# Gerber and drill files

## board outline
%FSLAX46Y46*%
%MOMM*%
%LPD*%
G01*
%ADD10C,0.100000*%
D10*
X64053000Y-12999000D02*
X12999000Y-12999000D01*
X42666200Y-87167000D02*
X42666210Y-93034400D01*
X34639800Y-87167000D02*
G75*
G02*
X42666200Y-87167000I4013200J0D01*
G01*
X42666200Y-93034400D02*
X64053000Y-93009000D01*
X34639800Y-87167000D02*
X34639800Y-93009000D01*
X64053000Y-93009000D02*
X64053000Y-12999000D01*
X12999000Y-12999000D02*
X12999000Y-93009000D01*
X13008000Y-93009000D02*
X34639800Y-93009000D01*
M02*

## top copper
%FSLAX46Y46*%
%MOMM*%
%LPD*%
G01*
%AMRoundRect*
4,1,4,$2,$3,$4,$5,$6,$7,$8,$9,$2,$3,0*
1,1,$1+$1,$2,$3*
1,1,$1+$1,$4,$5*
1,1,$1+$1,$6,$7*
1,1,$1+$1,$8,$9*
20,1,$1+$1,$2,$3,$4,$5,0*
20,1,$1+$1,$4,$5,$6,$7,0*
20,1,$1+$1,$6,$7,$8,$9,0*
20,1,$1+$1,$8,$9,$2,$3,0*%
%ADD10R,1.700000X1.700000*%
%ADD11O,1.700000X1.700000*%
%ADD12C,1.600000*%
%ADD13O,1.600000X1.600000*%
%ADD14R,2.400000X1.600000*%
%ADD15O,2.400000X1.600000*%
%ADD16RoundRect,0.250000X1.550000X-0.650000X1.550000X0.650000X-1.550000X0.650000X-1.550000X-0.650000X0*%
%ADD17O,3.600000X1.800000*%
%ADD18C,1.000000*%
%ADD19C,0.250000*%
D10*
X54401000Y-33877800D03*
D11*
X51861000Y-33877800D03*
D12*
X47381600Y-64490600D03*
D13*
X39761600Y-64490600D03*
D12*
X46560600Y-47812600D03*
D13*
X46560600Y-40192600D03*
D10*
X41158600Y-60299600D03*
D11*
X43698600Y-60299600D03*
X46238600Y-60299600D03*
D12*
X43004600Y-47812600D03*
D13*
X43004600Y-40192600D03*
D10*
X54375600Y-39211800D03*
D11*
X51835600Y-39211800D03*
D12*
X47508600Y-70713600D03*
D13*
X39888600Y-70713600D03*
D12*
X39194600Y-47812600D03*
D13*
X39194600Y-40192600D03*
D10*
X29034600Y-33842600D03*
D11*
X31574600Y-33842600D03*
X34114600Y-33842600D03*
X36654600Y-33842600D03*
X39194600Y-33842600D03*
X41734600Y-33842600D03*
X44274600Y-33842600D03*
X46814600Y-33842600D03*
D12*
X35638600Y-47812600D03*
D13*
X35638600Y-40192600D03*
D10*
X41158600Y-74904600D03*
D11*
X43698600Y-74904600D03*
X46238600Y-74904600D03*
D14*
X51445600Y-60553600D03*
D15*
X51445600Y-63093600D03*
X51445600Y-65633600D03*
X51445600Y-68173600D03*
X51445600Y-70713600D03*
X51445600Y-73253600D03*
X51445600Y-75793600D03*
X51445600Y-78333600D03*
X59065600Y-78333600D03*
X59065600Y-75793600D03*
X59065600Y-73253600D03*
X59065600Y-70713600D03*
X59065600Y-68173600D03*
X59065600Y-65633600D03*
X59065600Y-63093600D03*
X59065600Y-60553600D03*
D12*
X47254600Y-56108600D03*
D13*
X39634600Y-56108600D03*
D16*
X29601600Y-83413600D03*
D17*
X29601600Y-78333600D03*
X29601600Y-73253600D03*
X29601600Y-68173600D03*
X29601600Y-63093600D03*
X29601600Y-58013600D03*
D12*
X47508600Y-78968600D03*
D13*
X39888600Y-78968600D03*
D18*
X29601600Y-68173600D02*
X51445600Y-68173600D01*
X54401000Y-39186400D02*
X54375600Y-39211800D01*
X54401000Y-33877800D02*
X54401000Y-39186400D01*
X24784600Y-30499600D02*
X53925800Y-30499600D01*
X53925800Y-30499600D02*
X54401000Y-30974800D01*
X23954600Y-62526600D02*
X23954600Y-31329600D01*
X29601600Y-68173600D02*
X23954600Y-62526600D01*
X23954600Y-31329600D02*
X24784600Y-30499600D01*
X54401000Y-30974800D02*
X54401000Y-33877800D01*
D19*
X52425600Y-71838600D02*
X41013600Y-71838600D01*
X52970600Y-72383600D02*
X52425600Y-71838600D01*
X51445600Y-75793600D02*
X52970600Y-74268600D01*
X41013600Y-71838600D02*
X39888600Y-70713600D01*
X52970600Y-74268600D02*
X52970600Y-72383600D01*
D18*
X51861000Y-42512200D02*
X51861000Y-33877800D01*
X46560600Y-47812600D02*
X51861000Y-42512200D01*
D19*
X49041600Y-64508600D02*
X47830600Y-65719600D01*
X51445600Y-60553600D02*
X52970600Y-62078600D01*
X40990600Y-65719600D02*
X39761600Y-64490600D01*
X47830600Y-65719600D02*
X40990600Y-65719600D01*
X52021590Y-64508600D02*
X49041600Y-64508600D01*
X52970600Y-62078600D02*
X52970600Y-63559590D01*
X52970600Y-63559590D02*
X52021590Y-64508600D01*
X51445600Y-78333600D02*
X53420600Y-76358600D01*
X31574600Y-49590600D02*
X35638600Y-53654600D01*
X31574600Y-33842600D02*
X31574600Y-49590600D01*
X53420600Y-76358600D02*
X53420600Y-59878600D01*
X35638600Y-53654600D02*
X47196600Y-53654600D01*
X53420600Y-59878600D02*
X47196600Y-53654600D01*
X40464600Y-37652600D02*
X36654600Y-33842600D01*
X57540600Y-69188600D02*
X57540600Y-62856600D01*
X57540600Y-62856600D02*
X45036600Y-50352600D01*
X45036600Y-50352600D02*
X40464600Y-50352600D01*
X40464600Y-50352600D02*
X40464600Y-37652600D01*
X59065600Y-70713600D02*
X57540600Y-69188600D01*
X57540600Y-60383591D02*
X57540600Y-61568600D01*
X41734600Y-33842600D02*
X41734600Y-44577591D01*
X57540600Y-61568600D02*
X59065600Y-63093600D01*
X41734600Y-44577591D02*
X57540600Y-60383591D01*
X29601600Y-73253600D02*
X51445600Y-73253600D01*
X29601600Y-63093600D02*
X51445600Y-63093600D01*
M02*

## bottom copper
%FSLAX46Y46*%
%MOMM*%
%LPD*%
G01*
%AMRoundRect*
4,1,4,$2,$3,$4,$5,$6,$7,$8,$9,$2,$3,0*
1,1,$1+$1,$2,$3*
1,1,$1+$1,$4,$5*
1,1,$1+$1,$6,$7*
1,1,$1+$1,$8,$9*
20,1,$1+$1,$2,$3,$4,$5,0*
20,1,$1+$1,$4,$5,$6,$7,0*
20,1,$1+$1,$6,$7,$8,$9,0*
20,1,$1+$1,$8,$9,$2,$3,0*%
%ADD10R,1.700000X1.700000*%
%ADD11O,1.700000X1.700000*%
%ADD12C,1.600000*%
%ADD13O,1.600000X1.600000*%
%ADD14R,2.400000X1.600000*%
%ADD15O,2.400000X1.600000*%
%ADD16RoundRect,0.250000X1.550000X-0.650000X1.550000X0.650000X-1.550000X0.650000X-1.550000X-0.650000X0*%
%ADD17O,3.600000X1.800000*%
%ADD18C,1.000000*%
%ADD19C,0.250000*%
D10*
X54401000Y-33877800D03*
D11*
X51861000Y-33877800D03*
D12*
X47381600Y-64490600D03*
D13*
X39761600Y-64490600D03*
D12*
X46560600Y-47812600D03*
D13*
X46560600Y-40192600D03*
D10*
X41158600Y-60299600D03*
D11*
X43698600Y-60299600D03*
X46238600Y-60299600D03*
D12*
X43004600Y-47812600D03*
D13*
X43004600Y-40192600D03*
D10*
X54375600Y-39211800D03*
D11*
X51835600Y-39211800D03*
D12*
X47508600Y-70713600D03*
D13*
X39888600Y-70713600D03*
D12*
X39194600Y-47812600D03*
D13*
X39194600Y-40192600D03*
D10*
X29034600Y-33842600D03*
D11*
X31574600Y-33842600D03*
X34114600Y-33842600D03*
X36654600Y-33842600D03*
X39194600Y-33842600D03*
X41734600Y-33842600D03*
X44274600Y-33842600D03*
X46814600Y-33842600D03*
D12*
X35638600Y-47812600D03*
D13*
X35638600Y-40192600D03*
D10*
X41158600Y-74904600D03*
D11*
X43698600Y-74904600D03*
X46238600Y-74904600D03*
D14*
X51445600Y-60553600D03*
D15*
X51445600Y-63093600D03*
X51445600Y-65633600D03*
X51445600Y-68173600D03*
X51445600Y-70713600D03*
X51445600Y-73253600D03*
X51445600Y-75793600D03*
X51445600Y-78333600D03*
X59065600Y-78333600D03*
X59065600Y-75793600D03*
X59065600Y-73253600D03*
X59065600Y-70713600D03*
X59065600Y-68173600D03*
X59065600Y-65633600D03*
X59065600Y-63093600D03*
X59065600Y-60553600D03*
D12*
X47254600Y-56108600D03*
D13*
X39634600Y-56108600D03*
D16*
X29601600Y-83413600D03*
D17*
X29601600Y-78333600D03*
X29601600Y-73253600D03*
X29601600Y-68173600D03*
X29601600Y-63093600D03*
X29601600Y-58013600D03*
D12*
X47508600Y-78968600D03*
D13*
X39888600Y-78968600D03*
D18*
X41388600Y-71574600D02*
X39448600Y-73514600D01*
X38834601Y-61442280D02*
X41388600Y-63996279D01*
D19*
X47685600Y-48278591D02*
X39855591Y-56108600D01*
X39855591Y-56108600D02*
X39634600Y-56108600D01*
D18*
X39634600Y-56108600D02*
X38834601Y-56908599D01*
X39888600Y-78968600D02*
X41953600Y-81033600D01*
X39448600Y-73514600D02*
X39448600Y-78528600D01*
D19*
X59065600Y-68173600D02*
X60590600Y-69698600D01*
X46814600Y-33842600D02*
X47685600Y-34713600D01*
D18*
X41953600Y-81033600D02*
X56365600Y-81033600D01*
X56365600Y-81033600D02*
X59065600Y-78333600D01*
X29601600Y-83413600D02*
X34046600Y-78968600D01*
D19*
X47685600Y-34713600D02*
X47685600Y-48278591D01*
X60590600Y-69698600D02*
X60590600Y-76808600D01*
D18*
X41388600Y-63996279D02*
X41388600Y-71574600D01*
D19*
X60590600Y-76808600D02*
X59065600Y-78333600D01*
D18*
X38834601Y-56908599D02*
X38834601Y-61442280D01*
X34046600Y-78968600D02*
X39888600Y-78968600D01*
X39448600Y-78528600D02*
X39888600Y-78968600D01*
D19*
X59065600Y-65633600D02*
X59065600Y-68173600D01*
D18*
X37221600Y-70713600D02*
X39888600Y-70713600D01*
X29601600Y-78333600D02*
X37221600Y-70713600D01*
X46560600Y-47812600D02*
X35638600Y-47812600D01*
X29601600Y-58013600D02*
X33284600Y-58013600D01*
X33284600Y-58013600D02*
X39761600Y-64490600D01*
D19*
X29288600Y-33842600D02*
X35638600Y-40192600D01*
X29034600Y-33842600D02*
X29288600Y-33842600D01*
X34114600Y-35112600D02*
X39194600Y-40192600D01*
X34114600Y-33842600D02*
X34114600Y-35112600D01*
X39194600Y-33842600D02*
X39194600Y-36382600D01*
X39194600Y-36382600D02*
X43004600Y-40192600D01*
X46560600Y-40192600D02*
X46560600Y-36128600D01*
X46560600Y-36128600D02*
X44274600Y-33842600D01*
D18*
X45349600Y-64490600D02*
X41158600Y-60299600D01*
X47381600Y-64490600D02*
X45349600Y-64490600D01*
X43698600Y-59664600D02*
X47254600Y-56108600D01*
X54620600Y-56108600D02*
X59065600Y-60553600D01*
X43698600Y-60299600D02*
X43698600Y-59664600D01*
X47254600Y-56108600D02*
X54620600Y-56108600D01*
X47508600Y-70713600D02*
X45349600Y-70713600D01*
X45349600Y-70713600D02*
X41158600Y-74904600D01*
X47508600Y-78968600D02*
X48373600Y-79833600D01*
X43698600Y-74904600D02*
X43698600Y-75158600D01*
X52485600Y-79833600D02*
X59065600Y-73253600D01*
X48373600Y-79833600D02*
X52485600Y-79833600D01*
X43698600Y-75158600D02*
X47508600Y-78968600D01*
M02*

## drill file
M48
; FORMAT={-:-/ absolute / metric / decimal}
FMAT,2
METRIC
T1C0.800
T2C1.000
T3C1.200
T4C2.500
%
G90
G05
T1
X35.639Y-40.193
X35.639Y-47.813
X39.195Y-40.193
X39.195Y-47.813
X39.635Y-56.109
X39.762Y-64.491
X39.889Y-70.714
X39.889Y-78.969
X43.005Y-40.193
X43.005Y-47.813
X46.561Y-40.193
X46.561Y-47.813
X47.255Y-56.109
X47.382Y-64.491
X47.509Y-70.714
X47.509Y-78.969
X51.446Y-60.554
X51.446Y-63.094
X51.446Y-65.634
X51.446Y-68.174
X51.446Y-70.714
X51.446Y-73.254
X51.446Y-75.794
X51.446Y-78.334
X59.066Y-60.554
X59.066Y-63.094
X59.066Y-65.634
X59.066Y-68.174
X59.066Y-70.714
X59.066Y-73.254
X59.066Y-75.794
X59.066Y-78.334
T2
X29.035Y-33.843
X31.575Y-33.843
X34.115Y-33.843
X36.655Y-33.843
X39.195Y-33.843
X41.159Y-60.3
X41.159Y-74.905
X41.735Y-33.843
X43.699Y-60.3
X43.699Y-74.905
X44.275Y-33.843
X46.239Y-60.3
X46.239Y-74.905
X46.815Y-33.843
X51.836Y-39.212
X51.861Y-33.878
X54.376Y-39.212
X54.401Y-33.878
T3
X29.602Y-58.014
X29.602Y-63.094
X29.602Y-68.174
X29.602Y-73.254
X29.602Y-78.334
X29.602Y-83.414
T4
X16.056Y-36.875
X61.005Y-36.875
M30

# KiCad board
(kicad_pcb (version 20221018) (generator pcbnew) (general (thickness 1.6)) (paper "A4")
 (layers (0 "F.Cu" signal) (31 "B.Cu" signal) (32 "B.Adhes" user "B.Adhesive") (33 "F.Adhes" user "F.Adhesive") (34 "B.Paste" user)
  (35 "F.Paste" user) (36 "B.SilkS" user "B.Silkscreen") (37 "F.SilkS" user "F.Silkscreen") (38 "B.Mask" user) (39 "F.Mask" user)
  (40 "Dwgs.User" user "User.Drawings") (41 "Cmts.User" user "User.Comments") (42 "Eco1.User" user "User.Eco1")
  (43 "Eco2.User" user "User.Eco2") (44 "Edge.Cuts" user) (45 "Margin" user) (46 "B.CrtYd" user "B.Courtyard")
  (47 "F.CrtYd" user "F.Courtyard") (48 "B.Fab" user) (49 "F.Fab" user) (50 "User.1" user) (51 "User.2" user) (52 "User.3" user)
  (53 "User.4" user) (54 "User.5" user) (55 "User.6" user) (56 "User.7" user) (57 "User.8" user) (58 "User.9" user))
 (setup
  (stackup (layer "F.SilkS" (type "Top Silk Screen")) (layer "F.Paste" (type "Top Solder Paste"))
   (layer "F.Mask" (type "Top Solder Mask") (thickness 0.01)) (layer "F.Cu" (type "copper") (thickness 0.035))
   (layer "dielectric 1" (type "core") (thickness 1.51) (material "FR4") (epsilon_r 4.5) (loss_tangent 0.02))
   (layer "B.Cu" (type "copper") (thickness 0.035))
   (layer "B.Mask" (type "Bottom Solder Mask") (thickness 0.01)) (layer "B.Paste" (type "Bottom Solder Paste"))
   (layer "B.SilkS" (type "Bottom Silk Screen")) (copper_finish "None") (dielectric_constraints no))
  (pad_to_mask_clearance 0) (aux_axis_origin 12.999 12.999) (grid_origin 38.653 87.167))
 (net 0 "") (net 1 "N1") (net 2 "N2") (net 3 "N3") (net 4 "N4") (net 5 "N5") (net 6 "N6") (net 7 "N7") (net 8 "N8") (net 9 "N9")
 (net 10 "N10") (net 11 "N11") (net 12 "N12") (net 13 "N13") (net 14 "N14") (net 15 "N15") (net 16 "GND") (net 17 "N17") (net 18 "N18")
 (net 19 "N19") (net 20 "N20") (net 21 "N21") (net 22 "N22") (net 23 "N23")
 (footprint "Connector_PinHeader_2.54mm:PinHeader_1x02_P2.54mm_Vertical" (layer "F.Cu") (at 54.401 33.8778 -90)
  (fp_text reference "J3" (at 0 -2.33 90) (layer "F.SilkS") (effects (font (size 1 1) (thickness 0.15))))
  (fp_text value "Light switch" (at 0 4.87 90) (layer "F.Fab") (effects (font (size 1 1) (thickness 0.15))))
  (pad "1" thru_hole rect (at 0 0 270) (size 1.7 1.7) (drill 1) (layers "*.Cu" "*.Mask") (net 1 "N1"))
  (pad "2" thru_hole oval (at 0 2.54 270) (size 1.7 1.7) (drill 1) (layers "*.Cu" "*.Mask") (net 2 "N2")))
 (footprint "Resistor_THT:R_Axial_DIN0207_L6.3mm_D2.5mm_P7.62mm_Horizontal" (layer "F.Cu") (at 47.3816 64.4906 180)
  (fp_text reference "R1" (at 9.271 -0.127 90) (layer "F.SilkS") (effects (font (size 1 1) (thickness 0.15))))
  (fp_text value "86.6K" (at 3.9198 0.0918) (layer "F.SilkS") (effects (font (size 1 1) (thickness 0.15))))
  (pad "1" thru_hole circle (at 0 0 180) (size 1.6 1.6) (drill 0.8) (layers "*.Cu" "*.Mask") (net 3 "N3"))
  (pad "2" thru_hole oval (at 7.62 0 180) (size 1.6 1.6) (drill 0.8) (layers "*.Cu" "*.Mask") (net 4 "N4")))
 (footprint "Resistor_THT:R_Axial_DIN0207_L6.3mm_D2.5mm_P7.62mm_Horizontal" (layer "F.Cu") (at 46.5606 47.8126 90)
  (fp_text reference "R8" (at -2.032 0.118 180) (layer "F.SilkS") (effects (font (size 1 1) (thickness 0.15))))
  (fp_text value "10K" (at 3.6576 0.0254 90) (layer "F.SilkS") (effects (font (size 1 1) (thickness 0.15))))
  (pad "1" thru_hole circle (at 0 0 90) (size 1.6 1.6) (drill 0.8) (layers "*.Cu" "*.Mask") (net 2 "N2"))
  (pad "2" thru_hole oval (at 7.62 0 90) (size 1.6 1.6) (drill 0.8) (layers "*.Cu" "*.Mask") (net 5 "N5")))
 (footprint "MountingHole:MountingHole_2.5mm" (layer "F.Cu") (at 61.005 36.875)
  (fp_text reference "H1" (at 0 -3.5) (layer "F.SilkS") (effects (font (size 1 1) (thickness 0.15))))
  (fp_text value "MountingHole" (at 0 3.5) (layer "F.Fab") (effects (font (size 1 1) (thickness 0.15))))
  (pad "" np_thru_hole circle (at 0 0) (size 2.5 2.5) (drill 2.5) (layers "*.Cu" "*.Mask")))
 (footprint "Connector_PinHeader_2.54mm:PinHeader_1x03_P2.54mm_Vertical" (layer "F.Cu") (at 41.1586 60.2996 90)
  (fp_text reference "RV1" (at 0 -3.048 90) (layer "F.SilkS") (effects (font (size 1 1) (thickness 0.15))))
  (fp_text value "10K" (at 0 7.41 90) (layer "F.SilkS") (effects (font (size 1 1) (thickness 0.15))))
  (pad "1" thru_hole rect (at 0 0 90) (size 1.7 1.7) (drill 1) (layers "*.Cu" "*.Mask") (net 3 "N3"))
  (pad "2" thru_hole oval (at 0 2.54 90) (size 1.7 1.7) (drill 1) (layers "*.Cu" "*.Mask") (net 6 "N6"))
  (pad "3" thru_hole oval (at 0 5.08 90) (size 1.7 1.7) (drill 1) (layers "*.Cu" "*.Mask") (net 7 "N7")))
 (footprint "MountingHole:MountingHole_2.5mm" (layer "F.Cu") (at 16.056 36.875)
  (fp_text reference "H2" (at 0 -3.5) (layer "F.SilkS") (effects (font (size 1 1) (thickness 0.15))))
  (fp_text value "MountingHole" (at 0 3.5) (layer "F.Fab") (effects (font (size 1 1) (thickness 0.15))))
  (pad "" np_thru_hole circle (at 0 0) (size 2.5 2.5) (drill 2.5) (layers "*.Cu" "*.Mask")))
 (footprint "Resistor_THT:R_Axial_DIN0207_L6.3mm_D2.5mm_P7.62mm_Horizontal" (layer "F.Cu") (at 43.0046 47.8126 90)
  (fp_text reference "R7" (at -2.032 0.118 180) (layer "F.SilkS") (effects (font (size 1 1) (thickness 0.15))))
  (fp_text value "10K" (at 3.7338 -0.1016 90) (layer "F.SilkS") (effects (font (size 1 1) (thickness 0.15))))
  (pad "1" thru_hole circle (at 0 0 90) (size 1.6 1.6) (drill 0.8) (layers "*.Cu" "*.Mask") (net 2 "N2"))
  (pad "2" thru_hole oval (at 7.62 0 90) (size 1.6 1.6) (drill 0.8) (layers "*.Cu" "*.Mask") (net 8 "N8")))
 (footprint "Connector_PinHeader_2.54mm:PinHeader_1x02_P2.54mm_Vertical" (layer "F.Cu") (at 54.3756 39.2118 -90)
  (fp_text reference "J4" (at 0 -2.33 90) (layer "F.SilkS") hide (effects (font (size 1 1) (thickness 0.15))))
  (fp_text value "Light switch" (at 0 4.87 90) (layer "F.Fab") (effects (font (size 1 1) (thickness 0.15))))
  (pad "1" thru_hole rect (at 0 0 270) (size 1.7 1.7) (drill 1) (layers "*.Cu" "*.Mask") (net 1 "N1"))
  (pad "2" thru_hole oval (at 0 2.54 270) (size 1.7 1.7) (drill 1) (layers "*.Cu" "*.Mask") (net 2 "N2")))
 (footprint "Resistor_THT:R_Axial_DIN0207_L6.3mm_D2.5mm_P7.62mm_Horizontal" (layer "F.Cu") (at 47.5086 70.7136 180)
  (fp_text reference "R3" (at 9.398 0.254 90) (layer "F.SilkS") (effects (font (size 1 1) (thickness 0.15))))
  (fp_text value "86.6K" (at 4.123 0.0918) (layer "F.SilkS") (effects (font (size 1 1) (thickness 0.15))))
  (pad "1" thru_hole circle (at 0 0 180) (size 1.6 1.6) (drill 0.8) (layers "*.Cu" "*.Mask") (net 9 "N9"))
  (pad "2" thru_hole oval (at 7.62 0 180) (size 1.6 1.6) (drill 0.8) (layers "*.Cu" "*.Mask") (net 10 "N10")))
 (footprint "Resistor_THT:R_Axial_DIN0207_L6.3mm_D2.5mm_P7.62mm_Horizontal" (layer "F.Cu") (at 39.1946 47.8126 90)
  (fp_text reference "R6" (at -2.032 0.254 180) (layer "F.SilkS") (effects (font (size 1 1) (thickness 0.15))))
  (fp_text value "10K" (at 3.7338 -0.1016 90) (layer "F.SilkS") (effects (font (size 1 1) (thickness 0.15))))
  (pad "1" thru_hole circle (at 0 0 90) (size 1.6 1.6) (drill 0.8) (layers "*.Cu" "*.Mask") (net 2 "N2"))
  (pad "2" thru_hole oval (at 7.62 0 90) (size 1.6 1.6) (drill 0.8) (layers "*.Cu" "*.Mask") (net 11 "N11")))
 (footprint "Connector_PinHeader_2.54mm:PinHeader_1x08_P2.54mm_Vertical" (layer "F.Cu") (at 29.0346 33.8426 90)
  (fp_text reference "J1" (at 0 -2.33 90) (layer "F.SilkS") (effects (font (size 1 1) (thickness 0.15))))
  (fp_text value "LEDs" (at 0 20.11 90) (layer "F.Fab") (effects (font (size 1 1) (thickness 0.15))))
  (pad "1" thru_hole rect (at 0 0 90) (size 1.7 1.7) (drill 1) (layers "*.Cu" "*.Mask") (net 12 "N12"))
  (pad "2" thru_hole oval (at 0 2.54 90) (size 1.7 1.7) (drill 1) (layers "*.Cu" "*.Mask") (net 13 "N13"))
  (pad "3" thru_hole oval (at 0 5.08 90) (size 1.7 1.7) (drill 1) (layers "*.Cu" "*.Mask") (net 11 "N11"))
  (pad "4" thru_hole oval (at 0 7.62 90) (size 1.7 1.7) (drill 1) (layers "*.Cu" "*.Mask") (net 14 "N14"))
  (pad "5" thru_hole oval (at 0 10.16 90) (size 1.7 1.7) (drill 1) (layers "*.Cu" "*.Mask") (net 8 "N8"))
  (pad "6" thru_hole oval (at 0 12.7 90) (size 1.7 1.7) (drill 1) (layers "*.Cu" "*.Mask") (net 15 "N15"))
  (pad "7" thru_hole oval (at 0 15.24 90) (size 1.7 1.7) (drill 1) (layers "*.Cu" "*.Mask") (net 5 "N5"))
  (pad "8" thru_hole oval (at 0 17.78 90) (size 1.7 1.7) (drill 1) (layers "*.Cu" "*.Mask") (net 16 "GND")))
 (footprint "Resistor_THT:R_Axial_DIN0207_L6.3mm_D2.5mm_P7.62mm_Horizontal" (layer "F.Cu") (at 35.6386 47.8126 90)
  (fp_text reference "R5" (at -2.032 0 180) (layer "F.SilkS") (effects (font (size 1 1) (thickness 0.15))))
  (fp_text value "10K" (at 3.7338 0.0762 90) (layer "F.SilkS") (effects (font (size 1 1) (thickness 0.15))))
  (pad "1" thru_hole circle (at 0 0 90) (size 1.6 1.6) (drill 0.8) (layers "*.Cu" "*.Mask") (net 2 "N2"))
  (pad "2" thru_hole oval (at 7.62 0 90) (size 1.6 1.6) (drill 0.8) (layers "*.Cu" "*.Mask") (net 12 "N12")))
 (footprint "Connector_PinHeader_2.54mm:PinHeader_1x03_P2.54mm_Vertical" (layer "F.Cu") (at 41.1586 74.9046 90)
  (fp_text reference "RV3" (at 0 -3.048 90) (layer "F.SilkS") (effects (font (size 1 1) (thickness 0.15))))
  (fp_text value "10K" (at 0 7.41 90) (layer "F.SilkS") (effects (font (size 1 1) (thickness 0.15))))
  (pad "1" thru_hole rect (at 0 0 90) (size 1.7 1.7) (drill 1) (layers "*.Cu" "*.Mask") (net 9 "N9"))
  (pad "2" thru_hole oval (at 0 2.54 90) (size 1.7 1.7) (drill 1) (layers "*.Cu" "*.Mask") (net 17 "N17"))
  (pad "3" thru_hole oval (at 0 5.08 90) (size 1.7 1.7) (drill 1) (layers "*.Cu" "*.Mask") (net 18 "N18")))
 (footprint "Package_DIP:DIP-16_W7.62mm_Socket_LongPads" (layer "F.Cu") (at 51.4456 60.5536)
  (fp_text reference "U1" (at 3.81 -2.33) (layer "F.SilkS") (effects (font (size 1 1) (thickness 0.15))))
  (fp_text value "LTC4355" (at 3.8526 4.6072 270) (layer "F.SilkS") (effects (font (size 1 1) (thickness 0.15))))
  (pad "1" thru_hole rect (at 0 0) (size 2.4 1.6) (drill 0.8) (layers "*.Cu" "*.Mask") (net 4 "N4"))
  (pad "2" thru_hole oval (at 0 2.54) (size 2.4 1.6) (drill 0.8) (layers "*.Cu" "*.Mask") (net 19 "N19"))
  (pad "3" thru_hole oval (at 0 5.08) (size 2.4 1.6) (drill 0.8) (layers "*.Cu" "*.Mask") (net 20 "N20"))
  (pad "4" thru_hole oval (at 0 7.62) (size 2.4 1.6) (drill 0.8) (layers "*.Cu" "*.Mask") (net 1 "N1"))
  (pad "5" thru_hole oval (at 0 10.16) (size 2.4 1.6) (drill 0.8) (layers "*.Cu" "*.Mask") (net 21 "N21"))
  (pad "6" thru_hole oval (at 0 12.7) (size 2.4 1.6) (drill 0.8) (layers "*.Cu" "*.Mask") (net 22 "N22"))
  (pad "7" thru_hole oval (at 0 15.24) (size 2.4 1.6) (drill 0.8) (layers "*.Cu" "*.Mask") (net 10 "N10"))
  (pad "8" thru_hole oval (at 0 17.78) (size 2.4 1.6) (drill 0.8) (layers "*.Cu" "*.Mask") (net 13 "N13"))
  (pad "9" thru_hole oval (at 7.62 17.78) (size 2.4 1.6) (drill 0.8) (layers "*.Cu" "*.Mask") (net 16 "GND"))
  (pad "10" thru_hole oval (at 7.62 15.24) (size 2.4 1.6) (drill 0.8) (layers "*.Cu" "*.Mask") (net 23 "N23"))
  (pad "11" thru_hole oval (at 7.62 12.7) (size 2.4 1.6) (drill 0.8) (layers "*.Cu" "*.Mask") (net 17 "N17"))
  (pad "12" thru_hole oval (at 7.62 10.16) (size 2.4 1.6) (drill 0.8) (layers "*.Cu" "*.Mask") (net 14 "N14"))
  (pad "13" thru_hole oval (at 7.62 7.62) (size 2.4 1.6) (drill 0.8) (layers "*.Cu" "*.Mask") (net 16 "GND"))
  (pad "14" thru_hole oval (at 7.62 5.08) (size 2.4 1.6) (drill 0.8) (layers "*.Cu" "*.Mask") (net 16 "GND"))
  (pad "15" thru_hole oval (at 7.62 2.54) (size 2.4 1.6) (drill 0.8) (layers "*.Cu" "*.Mask") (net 15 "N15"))
  (pad "16" thru_hole oval (at 7.62 0) (size 2.4 1.6) (drill 0.8) (layers "*.Cu" "*.Mask") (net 6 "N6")))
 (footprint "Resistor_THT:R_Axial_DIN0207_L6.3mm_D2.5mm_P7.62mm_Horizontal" (layer "F.Cu") (at 47.2546 56.1086 180)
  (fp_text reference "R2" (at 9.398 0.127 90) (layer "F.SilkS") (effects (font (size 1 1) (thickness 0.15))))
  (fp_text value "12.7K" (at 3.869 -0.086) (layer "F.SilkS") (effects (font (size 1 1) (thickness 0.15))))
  (pad "1" thru_hole circle (at 0 0 180) (size 1.6 1.6) (drill 0.8) (layers "*.Cu" "*.Mask") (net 6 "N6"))
  (pad "2" thru_hole oval (at 7.62 0 180) (size 1.6 1.6) (drill 0.8) (layers "*.Cu" "*.Mask") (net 16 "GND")))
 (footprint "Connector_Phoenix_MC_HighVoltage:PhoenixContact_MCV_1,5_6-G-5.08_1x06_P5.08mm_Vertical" (layer "F.Cu") (at 29.6016 83.4136 90)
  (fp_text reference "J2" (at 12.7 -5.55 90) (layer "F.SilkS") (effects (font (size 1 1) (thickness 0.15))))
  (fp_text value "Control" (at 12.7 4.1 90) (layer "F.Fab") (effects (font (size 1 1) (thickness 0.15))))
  (pad "1" thru_hole roundrect (at 0 0 90) (size 1.8 3.6) (drill 1.2) (layers "*.Cu" "*.Mask") (roundrect_rratio 0.1388888889)
   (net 16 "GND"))
  (pad "2" thru_hole oval (at 5.08 0 90) (size 1.8 3.6) (drill 1.2) (layers "*.Cu" "*.Mask") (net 10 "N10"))
  (pad "3" thru_hole oval (at 10.16 0 90) (size 1.8 3.6) (drill 1.2) (layers "*.Cu" "*.Mask") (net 22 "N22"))
  (pad "4" thru_hole oval (at 15.24 0 90) (size 1.8 3.6) (drill 1.2) (layers "*.Cu" "*.Mask") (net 1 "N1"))
  (pad "5" thru_hole oval (at 20.32 0 90) (size 1.8 3.6) (drill 1.2) (layers "*.Cu" "*.Mask") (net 19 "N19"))
  (pad "6" thru_hole oval (at 25.4 0 90) (size 1.8 3.6) (drill 1.2) (layers "*.Cu" "*.Mask") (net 4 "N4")))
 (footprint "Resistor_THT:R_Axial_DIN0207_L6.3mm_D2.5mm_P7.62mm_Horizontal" (layer "F.Cu") (at 47.5086 78.9686 180)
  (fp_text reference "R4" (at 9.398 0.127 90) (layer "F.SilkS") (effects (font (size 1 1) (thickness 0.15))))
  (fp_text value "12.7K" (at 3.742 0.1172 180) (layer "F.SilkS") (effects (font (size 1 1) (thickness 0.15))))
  (pad "1" thru_hole circle (at 0 0 180) (size 1.6 1.6) (drill 0.8) (layers "*.Cu" "*.Mask") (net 17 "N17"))
  (pad "2" thru_hole oval (at 7.62 0 180) (size 1.6 1.6) (drill 0.8) (layers "*.Cu" "*.Mask") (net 16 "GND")))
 (gr_line (start 64.053 12.999) (end 12.999 12.999) (stroke (width 0.1) (type default)) (layer "Edge.Cuts"))
 (gr_line (start 42.6662 87.167) (end 42.66621 93.0344) (stroke (width 0.1) (type default)) (layer "Edge.Cuts"))
 (gr_arc (start 34.6398 87.167) (mid 38.653 83.1538) (end 42.6662 87.167) (stroke (width 0.1) (type default)) (layer "Edge.Cuts"))
 (gr_line (start 42.6662 93.0344) (end 64.053 93.009) (stroke (width 0.1) (type default)) (layer "Edge.Cuts"))
 (gr_line (start 34.6398 87.167) (end 34.6398 93.009) (stroke (width 0.1) (type default)) (layer "Edge.Cuts"))
 (gr_line (start 64.053 93.009) (end 64.053 12.999) (stroke (width 0.1) (type default)) (layer "Edge.Cuts"))
 (gr_line (start 12.999 12.999) (end 12.999 93.009) (stroke (width 0.1) (type default)) (layer "Edge.Cuts"))
 (gr_line (start 13.008 93.009) (end 34.6398 93.009) (stroke (width 0.1) (type default)) (layer "Edge.Cuts"))
 (segment (start 41.3886 71.5746) (end 39.4486 73.5146) (width 1) (layer "B.Cu") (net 16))
 (segment (start 38.834601 61.44228) (end 41.3886 63.996279) (width 1) (layer "B.Cu") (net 16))
 (segment (start 47.6856 48.278591) (end 39.855591 56.1086) (width 0.25) (layer "B.Cu") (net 16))
 (segment (start 39.855591 56.1086) (end 39.6346 56.1086) (width 0.25) (layer "B.Cu") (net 16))
 (segment (start 39.6346 56.1086) (end 38.834601 56.908599) (width 1) (layer "B.Cu") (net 16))
 (segment (start 39.8886 78.9686) (end 41.9536 81.0336) (width 1) (layer "B.Cu") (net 16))
 (segment (start 39.4486 73.5146) (end 39.4486 78.5286) (width 1) (layer "B.Cu") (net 16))
 (segment (start 59.0656 68.1736) (end 60.5906 69.6986) (width 0.25) (layer "B.Cu") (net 16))
 (segment (start 46.8146 33.8426) (end 47.6856 34.7136) (width 0.25) (layer "B.Cu") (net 16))
 (segment (start 41.9536 81.0336) (end 56.3656 81.0336) (width 1) (layer "B.Cu") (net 16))
 (segment (start 56.3656 81.0336) (end 59.0656 78.3336) (width 1) (layer "B.Cu") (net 16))
 (segment (start 29.6016 83.4136) (end 34.0466 78.9686) (width 1) (layer "B.Cu") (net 16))
 (segment (start 47.6856 34.7136) (end 47.6856 48.278591) (width 0.25) (layer "B.Cu") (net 16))
 (segment (start 60.5906 69.6986) (end 60.5906 76.8086) (width 0.25) (layer "B.Cu") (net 16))
 (segment (start 41.3886 63.996279) (end 41.3886 71.5746) (width 1) (layer "B.Cu") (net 16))
 (segment (start 60.5906 76.8086) (end 59.0656 78.3336) (width 0.25) (layer "B.Cu") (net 16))
 (segment (start 38.834601 56.908599) (end 38.834601 61.44228) (width 1) (layer "B.Cu") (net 16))
 (segment (start 34.0466 78.9686) (end 39.8886 78.9686) (width 1) (layer "B.Cu") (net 16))
 (segment (start 39.4486 78.5286) (end 39.8886 78.9686) (width 1) (layer "B.Cu") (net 16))
 (segment (start 59.0656 65.6336) (end 59.0656 68.1736) (width 0.25) (layer "B.Cu") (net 16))
 (segment (start 29.6016 68.1736) (end 51.4456 68.1736) (width 1) (layer "F.Cu") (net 1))
 (segment (start 54.401 39.1864) (end 54.3756 39.2118) (width 1) (layer "F.Cu") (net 1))
 (segment (start 54.401 33.8778) (end 54.401 39.1864) (width 1) (layer "F.Cu") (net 1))
 (segment (start 24.7846 30.4996) (end 53.9258 30.4996) (width 1) (layer "F.Cu") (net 1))
 (segment (start 53.9258 30.4996) (end 54.401 30.9748) (width 1) (layer "F.Cu") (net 1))
 (segment (start 23.9546 62.5266) (end 23.9546 31.3296) (width 1) (layer "F.Cu") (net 1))
 (segment (start 29.6016 68.1736) (end 23.9546 62.5266) (width 1) (layer "F.Cu") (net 1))
 (segment (start 23.9546 31.3296) (end 24.7846 30.4996) (width 1) (layer "F.Cu") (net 1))
 (segment (start 54.401 30.9748) (end 54.401 33.8778) (width 1) (layer "F.Cu") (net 1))
 (segment (start 52.4256 71.8386) (end 41.0136 71.8386) (width 0.25) (layer "F.Cu") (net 10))
 (segment (start 52.9706 72.3836) (end 52.4256 71.8386) (width 0.25) (layer "F.Cu") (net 10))
 (segment (start 51.4456 75.7936) (end 52.9706 74.2686) (width 0.25) (layer "F.Cu") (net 10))
 (segment (start 41.0136 71.8386) (end 39.8886 70.7136) (width 0.25) (layer "F.Cu") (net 10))
 (segment (start 52.9706 74.2686) (end 52.9706 72.3836) (width 0.25) (layer "F.Cu") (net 10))
 (segment (start 37.2216 70.7136) (end 39.8886 70.7136) (width 1) (layer "B.Cu") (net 10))
 (segment (start 29.6016 78.3336) (end 37.2216 70.7136) (width 1) (layer "B.Cu") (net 10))
 (segment (start 51.861 42.5122) (end 51.861 33.8778) (width 1) (layer "F.Cu") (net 2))
 (segment (start 46.5606 47.8126) (end 51.861 42.5122) (width 1) (layer "F.Cu") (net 2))
 (segment (start 46.5606 47.8126) (end 35.6386 47.8126) (width 1) (layer "B.Cu") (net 2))
 (segment (start 49.0416 64.5086) (end 47.8306 65.7196) (width 0.25) (layer "F.Cu") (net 4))
 (segment (start 51.4456 60.5536) (end 52.9706 62.0786) (width 0.25) (layer "F.Cu") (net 4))
 (segment (start 40.9906 65.7196) (end 39.7616 64.4906) (width 0.25) (layer "F.Cu") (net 4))
 (segment (start 47.8306 65.7196) (end 40.9906 65.7196) (width 0.25) (layer "F.Cu") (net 4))
 (segment (start 52.02159 64.5086) (end 49.0416 64.5086) (width 0.25) (layer "F.Cu") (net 4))
 (segment (start 52.9706 62.0786) (end 52.9706 63.55959) (width 0.25) (layer "F.Cu") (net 4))
 (segment (start 52.9706 63.55959) (end 52.02159 64.5086) (width 0.25) (layer "F.Cu") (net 4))
 (segment (start 29.6016 58.0136) (end 33.2846 58.0136) (width 1) (layer "B.Cu") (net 4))
 (segment (start 33.2846 58.0136) (end 39.7616 64.4906) (width 1) (layer "B.Cu") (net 4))
 (segment (start 29.2886 33.8426) (end 35.6386 40.1926) (width 0.25) (layer "B.Cu") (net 12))
 (segment (start 29.0346 33.8426) (end 29.2886 33.8426) (width 0.25) (layer "B.Cu") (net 12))
 (segment (start 51.4456 78.3336) (end 53.4206 76.3586) (width 0.25) (layer "F.Cu") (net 13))
 (segment (start 31.5746 49.5906) (end 35.6386 53.6546) (width 0.25) (layer "F.Cu") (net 13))
 (segment (start 31.5746 33.8426) (end 31.5746 49.5906) (width 0.25) (layer "F.Cu") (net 13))
 (segment (start 53.4206 76.3586) (end 53.4206 59.8786) (width 0.25) (layer "F.Cu") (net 13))
 (segment (start 35.6386 53.6546) (end 47.1966 53.6546) (width 0.25) (layer "F.Cu") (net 13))
 (segment (start 53.4206 59.8786) (end 47.1966 53.6546) (width 0.25) (layer "F.Cu") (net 13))
 (segment (start 34.1146 35.1126) (end 39.1946 40.1926) (width 0.25) (layer "B.Cu") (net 11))
 (segment (start 34.1146 33.8426) (end 34.1146 35.1126) (width 0.25) (layer "B.Cu") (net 11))
 (segment (start 40.4646 37.6526) (end 36.6546 33.8426) (width 0.25) (layer "F.Cu") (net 14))
 (segment (start 57.5406 69.1886) (end 57.5406 62.8566) (width 0.25) (layer "F.Cu") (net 14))
 (segment (start 57.5406 62.8566) (end 45.0366 50.3526) (width 0.25) (layer "F.Cu") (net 14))
 (segment (start 45.0366 50.3526) (end 40.4646 50.3526) (width 0.25) (layer "F.Cu") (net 14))
 (segment (start 40.4646 50.3526) (end 40.4646 37.6526) (width 0.25) (layer "F.Cu") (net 14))
 (segment (start 59.0656 70.7136) (end 57.5406 69.1886) (width 0.25) (layer "F.Cu") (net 14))
 (segment (start 39.1946 33.8426) (end 39.1946 36.3826) (width 0.25) (layer "B.Cu") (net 8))
 (segment (start 39.1946 36.3826) (end 43.0046 40.1926) (width 0.25) (layer "B.Cu") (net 8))
 (segment (start 57.5406 60.383591) (end 57.5406 61.5686) (width 0.25) (layer "F.Cu") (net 15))
 (segment (start 41.7346 33.8426) (end 41.7346 44.577591) (width 0.25) (layer "F.Cu") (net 15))
 (segment (start 57.5406 61.5686) (end 59.0656 63.0936) (width 0.25) (layer "F.Cu") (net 15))
 (segment (start 41.7346 44.577591) (end 57.5406 60.383591) (width 0.25) (layer "F.Cu") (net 15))
 (segment (start 46.5606 40.1926) (end 46.5606 36.1286) (width 0.25) (layer "B.Cu") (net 5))
 (segment (start 46.5606 36.1286) (end 44.2746 33.8426) (width 0.25) (layer "B.Cu") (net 5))
 (segment (start 29.6016 73.2536) (end 51.4456 73.2536) (width 0.25) (layer "F.Cu") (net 22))
 (segment (start 29.6016 63.0936) (end 51.4456 63.0936) (width 0.25) (layer "F.Cu") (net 19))
 (segment (start 45.3496 64.4906) (end 41.1586 60.2996) (width 1) (layer "B.Cu") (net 3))
 (segment (start 47.3816 64.4906) (end 45.3496 64.4906) (width 1) (layer "B.Cu") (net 3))
 (segment (start 43.6986 59.6646) (end 47.2546 56.1086) (width 1) (layer "B.Cu") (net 6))
 (segment (start 54.6206 56.1086) (end 59.0656 60.5536) (width 1) (layer "B.Cu") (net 6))
 (segment (start 43.6986 60.2996) (end 43.6986 59.6646) (width 1) (layer "B.Cu") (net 6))
 (segment (start 47.2546 56.1086) (end 54.6206 56.1086) (width 1) (layer "B.Cu") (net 6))
 (segment (start 47.5086 70.7136) (end 45.3496 70.7136) (width 1) (layer "B.Cu") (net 9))
 (segment (start 45.3496 70.7136) (end 41.1586 74.9046) (width 1) (layer "B.Cu") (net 9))
 (segment (start 47.5086 78.9686) (end 48.3736 79.8336) (width 1) (layer "B.Cu") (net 17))
 (segment (start 43.6986 74.9046) (end 43.6986 75.1586) (width 1) (layer "B.Cu") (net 17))
 (segment (start 52.4856 79.8336) (end 59.0656 73.2536) (width 1) (layer "B.Cu") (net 17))
 (segment (start 48.3736 79.8336) (end 52.4856 79.8336) (width 1) (layer "B.Cu") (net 17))
 (segment (start 43.6986 75.1586) (end 47.5086 78.9686) (width 1) (layer "B.Cu") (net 17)))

